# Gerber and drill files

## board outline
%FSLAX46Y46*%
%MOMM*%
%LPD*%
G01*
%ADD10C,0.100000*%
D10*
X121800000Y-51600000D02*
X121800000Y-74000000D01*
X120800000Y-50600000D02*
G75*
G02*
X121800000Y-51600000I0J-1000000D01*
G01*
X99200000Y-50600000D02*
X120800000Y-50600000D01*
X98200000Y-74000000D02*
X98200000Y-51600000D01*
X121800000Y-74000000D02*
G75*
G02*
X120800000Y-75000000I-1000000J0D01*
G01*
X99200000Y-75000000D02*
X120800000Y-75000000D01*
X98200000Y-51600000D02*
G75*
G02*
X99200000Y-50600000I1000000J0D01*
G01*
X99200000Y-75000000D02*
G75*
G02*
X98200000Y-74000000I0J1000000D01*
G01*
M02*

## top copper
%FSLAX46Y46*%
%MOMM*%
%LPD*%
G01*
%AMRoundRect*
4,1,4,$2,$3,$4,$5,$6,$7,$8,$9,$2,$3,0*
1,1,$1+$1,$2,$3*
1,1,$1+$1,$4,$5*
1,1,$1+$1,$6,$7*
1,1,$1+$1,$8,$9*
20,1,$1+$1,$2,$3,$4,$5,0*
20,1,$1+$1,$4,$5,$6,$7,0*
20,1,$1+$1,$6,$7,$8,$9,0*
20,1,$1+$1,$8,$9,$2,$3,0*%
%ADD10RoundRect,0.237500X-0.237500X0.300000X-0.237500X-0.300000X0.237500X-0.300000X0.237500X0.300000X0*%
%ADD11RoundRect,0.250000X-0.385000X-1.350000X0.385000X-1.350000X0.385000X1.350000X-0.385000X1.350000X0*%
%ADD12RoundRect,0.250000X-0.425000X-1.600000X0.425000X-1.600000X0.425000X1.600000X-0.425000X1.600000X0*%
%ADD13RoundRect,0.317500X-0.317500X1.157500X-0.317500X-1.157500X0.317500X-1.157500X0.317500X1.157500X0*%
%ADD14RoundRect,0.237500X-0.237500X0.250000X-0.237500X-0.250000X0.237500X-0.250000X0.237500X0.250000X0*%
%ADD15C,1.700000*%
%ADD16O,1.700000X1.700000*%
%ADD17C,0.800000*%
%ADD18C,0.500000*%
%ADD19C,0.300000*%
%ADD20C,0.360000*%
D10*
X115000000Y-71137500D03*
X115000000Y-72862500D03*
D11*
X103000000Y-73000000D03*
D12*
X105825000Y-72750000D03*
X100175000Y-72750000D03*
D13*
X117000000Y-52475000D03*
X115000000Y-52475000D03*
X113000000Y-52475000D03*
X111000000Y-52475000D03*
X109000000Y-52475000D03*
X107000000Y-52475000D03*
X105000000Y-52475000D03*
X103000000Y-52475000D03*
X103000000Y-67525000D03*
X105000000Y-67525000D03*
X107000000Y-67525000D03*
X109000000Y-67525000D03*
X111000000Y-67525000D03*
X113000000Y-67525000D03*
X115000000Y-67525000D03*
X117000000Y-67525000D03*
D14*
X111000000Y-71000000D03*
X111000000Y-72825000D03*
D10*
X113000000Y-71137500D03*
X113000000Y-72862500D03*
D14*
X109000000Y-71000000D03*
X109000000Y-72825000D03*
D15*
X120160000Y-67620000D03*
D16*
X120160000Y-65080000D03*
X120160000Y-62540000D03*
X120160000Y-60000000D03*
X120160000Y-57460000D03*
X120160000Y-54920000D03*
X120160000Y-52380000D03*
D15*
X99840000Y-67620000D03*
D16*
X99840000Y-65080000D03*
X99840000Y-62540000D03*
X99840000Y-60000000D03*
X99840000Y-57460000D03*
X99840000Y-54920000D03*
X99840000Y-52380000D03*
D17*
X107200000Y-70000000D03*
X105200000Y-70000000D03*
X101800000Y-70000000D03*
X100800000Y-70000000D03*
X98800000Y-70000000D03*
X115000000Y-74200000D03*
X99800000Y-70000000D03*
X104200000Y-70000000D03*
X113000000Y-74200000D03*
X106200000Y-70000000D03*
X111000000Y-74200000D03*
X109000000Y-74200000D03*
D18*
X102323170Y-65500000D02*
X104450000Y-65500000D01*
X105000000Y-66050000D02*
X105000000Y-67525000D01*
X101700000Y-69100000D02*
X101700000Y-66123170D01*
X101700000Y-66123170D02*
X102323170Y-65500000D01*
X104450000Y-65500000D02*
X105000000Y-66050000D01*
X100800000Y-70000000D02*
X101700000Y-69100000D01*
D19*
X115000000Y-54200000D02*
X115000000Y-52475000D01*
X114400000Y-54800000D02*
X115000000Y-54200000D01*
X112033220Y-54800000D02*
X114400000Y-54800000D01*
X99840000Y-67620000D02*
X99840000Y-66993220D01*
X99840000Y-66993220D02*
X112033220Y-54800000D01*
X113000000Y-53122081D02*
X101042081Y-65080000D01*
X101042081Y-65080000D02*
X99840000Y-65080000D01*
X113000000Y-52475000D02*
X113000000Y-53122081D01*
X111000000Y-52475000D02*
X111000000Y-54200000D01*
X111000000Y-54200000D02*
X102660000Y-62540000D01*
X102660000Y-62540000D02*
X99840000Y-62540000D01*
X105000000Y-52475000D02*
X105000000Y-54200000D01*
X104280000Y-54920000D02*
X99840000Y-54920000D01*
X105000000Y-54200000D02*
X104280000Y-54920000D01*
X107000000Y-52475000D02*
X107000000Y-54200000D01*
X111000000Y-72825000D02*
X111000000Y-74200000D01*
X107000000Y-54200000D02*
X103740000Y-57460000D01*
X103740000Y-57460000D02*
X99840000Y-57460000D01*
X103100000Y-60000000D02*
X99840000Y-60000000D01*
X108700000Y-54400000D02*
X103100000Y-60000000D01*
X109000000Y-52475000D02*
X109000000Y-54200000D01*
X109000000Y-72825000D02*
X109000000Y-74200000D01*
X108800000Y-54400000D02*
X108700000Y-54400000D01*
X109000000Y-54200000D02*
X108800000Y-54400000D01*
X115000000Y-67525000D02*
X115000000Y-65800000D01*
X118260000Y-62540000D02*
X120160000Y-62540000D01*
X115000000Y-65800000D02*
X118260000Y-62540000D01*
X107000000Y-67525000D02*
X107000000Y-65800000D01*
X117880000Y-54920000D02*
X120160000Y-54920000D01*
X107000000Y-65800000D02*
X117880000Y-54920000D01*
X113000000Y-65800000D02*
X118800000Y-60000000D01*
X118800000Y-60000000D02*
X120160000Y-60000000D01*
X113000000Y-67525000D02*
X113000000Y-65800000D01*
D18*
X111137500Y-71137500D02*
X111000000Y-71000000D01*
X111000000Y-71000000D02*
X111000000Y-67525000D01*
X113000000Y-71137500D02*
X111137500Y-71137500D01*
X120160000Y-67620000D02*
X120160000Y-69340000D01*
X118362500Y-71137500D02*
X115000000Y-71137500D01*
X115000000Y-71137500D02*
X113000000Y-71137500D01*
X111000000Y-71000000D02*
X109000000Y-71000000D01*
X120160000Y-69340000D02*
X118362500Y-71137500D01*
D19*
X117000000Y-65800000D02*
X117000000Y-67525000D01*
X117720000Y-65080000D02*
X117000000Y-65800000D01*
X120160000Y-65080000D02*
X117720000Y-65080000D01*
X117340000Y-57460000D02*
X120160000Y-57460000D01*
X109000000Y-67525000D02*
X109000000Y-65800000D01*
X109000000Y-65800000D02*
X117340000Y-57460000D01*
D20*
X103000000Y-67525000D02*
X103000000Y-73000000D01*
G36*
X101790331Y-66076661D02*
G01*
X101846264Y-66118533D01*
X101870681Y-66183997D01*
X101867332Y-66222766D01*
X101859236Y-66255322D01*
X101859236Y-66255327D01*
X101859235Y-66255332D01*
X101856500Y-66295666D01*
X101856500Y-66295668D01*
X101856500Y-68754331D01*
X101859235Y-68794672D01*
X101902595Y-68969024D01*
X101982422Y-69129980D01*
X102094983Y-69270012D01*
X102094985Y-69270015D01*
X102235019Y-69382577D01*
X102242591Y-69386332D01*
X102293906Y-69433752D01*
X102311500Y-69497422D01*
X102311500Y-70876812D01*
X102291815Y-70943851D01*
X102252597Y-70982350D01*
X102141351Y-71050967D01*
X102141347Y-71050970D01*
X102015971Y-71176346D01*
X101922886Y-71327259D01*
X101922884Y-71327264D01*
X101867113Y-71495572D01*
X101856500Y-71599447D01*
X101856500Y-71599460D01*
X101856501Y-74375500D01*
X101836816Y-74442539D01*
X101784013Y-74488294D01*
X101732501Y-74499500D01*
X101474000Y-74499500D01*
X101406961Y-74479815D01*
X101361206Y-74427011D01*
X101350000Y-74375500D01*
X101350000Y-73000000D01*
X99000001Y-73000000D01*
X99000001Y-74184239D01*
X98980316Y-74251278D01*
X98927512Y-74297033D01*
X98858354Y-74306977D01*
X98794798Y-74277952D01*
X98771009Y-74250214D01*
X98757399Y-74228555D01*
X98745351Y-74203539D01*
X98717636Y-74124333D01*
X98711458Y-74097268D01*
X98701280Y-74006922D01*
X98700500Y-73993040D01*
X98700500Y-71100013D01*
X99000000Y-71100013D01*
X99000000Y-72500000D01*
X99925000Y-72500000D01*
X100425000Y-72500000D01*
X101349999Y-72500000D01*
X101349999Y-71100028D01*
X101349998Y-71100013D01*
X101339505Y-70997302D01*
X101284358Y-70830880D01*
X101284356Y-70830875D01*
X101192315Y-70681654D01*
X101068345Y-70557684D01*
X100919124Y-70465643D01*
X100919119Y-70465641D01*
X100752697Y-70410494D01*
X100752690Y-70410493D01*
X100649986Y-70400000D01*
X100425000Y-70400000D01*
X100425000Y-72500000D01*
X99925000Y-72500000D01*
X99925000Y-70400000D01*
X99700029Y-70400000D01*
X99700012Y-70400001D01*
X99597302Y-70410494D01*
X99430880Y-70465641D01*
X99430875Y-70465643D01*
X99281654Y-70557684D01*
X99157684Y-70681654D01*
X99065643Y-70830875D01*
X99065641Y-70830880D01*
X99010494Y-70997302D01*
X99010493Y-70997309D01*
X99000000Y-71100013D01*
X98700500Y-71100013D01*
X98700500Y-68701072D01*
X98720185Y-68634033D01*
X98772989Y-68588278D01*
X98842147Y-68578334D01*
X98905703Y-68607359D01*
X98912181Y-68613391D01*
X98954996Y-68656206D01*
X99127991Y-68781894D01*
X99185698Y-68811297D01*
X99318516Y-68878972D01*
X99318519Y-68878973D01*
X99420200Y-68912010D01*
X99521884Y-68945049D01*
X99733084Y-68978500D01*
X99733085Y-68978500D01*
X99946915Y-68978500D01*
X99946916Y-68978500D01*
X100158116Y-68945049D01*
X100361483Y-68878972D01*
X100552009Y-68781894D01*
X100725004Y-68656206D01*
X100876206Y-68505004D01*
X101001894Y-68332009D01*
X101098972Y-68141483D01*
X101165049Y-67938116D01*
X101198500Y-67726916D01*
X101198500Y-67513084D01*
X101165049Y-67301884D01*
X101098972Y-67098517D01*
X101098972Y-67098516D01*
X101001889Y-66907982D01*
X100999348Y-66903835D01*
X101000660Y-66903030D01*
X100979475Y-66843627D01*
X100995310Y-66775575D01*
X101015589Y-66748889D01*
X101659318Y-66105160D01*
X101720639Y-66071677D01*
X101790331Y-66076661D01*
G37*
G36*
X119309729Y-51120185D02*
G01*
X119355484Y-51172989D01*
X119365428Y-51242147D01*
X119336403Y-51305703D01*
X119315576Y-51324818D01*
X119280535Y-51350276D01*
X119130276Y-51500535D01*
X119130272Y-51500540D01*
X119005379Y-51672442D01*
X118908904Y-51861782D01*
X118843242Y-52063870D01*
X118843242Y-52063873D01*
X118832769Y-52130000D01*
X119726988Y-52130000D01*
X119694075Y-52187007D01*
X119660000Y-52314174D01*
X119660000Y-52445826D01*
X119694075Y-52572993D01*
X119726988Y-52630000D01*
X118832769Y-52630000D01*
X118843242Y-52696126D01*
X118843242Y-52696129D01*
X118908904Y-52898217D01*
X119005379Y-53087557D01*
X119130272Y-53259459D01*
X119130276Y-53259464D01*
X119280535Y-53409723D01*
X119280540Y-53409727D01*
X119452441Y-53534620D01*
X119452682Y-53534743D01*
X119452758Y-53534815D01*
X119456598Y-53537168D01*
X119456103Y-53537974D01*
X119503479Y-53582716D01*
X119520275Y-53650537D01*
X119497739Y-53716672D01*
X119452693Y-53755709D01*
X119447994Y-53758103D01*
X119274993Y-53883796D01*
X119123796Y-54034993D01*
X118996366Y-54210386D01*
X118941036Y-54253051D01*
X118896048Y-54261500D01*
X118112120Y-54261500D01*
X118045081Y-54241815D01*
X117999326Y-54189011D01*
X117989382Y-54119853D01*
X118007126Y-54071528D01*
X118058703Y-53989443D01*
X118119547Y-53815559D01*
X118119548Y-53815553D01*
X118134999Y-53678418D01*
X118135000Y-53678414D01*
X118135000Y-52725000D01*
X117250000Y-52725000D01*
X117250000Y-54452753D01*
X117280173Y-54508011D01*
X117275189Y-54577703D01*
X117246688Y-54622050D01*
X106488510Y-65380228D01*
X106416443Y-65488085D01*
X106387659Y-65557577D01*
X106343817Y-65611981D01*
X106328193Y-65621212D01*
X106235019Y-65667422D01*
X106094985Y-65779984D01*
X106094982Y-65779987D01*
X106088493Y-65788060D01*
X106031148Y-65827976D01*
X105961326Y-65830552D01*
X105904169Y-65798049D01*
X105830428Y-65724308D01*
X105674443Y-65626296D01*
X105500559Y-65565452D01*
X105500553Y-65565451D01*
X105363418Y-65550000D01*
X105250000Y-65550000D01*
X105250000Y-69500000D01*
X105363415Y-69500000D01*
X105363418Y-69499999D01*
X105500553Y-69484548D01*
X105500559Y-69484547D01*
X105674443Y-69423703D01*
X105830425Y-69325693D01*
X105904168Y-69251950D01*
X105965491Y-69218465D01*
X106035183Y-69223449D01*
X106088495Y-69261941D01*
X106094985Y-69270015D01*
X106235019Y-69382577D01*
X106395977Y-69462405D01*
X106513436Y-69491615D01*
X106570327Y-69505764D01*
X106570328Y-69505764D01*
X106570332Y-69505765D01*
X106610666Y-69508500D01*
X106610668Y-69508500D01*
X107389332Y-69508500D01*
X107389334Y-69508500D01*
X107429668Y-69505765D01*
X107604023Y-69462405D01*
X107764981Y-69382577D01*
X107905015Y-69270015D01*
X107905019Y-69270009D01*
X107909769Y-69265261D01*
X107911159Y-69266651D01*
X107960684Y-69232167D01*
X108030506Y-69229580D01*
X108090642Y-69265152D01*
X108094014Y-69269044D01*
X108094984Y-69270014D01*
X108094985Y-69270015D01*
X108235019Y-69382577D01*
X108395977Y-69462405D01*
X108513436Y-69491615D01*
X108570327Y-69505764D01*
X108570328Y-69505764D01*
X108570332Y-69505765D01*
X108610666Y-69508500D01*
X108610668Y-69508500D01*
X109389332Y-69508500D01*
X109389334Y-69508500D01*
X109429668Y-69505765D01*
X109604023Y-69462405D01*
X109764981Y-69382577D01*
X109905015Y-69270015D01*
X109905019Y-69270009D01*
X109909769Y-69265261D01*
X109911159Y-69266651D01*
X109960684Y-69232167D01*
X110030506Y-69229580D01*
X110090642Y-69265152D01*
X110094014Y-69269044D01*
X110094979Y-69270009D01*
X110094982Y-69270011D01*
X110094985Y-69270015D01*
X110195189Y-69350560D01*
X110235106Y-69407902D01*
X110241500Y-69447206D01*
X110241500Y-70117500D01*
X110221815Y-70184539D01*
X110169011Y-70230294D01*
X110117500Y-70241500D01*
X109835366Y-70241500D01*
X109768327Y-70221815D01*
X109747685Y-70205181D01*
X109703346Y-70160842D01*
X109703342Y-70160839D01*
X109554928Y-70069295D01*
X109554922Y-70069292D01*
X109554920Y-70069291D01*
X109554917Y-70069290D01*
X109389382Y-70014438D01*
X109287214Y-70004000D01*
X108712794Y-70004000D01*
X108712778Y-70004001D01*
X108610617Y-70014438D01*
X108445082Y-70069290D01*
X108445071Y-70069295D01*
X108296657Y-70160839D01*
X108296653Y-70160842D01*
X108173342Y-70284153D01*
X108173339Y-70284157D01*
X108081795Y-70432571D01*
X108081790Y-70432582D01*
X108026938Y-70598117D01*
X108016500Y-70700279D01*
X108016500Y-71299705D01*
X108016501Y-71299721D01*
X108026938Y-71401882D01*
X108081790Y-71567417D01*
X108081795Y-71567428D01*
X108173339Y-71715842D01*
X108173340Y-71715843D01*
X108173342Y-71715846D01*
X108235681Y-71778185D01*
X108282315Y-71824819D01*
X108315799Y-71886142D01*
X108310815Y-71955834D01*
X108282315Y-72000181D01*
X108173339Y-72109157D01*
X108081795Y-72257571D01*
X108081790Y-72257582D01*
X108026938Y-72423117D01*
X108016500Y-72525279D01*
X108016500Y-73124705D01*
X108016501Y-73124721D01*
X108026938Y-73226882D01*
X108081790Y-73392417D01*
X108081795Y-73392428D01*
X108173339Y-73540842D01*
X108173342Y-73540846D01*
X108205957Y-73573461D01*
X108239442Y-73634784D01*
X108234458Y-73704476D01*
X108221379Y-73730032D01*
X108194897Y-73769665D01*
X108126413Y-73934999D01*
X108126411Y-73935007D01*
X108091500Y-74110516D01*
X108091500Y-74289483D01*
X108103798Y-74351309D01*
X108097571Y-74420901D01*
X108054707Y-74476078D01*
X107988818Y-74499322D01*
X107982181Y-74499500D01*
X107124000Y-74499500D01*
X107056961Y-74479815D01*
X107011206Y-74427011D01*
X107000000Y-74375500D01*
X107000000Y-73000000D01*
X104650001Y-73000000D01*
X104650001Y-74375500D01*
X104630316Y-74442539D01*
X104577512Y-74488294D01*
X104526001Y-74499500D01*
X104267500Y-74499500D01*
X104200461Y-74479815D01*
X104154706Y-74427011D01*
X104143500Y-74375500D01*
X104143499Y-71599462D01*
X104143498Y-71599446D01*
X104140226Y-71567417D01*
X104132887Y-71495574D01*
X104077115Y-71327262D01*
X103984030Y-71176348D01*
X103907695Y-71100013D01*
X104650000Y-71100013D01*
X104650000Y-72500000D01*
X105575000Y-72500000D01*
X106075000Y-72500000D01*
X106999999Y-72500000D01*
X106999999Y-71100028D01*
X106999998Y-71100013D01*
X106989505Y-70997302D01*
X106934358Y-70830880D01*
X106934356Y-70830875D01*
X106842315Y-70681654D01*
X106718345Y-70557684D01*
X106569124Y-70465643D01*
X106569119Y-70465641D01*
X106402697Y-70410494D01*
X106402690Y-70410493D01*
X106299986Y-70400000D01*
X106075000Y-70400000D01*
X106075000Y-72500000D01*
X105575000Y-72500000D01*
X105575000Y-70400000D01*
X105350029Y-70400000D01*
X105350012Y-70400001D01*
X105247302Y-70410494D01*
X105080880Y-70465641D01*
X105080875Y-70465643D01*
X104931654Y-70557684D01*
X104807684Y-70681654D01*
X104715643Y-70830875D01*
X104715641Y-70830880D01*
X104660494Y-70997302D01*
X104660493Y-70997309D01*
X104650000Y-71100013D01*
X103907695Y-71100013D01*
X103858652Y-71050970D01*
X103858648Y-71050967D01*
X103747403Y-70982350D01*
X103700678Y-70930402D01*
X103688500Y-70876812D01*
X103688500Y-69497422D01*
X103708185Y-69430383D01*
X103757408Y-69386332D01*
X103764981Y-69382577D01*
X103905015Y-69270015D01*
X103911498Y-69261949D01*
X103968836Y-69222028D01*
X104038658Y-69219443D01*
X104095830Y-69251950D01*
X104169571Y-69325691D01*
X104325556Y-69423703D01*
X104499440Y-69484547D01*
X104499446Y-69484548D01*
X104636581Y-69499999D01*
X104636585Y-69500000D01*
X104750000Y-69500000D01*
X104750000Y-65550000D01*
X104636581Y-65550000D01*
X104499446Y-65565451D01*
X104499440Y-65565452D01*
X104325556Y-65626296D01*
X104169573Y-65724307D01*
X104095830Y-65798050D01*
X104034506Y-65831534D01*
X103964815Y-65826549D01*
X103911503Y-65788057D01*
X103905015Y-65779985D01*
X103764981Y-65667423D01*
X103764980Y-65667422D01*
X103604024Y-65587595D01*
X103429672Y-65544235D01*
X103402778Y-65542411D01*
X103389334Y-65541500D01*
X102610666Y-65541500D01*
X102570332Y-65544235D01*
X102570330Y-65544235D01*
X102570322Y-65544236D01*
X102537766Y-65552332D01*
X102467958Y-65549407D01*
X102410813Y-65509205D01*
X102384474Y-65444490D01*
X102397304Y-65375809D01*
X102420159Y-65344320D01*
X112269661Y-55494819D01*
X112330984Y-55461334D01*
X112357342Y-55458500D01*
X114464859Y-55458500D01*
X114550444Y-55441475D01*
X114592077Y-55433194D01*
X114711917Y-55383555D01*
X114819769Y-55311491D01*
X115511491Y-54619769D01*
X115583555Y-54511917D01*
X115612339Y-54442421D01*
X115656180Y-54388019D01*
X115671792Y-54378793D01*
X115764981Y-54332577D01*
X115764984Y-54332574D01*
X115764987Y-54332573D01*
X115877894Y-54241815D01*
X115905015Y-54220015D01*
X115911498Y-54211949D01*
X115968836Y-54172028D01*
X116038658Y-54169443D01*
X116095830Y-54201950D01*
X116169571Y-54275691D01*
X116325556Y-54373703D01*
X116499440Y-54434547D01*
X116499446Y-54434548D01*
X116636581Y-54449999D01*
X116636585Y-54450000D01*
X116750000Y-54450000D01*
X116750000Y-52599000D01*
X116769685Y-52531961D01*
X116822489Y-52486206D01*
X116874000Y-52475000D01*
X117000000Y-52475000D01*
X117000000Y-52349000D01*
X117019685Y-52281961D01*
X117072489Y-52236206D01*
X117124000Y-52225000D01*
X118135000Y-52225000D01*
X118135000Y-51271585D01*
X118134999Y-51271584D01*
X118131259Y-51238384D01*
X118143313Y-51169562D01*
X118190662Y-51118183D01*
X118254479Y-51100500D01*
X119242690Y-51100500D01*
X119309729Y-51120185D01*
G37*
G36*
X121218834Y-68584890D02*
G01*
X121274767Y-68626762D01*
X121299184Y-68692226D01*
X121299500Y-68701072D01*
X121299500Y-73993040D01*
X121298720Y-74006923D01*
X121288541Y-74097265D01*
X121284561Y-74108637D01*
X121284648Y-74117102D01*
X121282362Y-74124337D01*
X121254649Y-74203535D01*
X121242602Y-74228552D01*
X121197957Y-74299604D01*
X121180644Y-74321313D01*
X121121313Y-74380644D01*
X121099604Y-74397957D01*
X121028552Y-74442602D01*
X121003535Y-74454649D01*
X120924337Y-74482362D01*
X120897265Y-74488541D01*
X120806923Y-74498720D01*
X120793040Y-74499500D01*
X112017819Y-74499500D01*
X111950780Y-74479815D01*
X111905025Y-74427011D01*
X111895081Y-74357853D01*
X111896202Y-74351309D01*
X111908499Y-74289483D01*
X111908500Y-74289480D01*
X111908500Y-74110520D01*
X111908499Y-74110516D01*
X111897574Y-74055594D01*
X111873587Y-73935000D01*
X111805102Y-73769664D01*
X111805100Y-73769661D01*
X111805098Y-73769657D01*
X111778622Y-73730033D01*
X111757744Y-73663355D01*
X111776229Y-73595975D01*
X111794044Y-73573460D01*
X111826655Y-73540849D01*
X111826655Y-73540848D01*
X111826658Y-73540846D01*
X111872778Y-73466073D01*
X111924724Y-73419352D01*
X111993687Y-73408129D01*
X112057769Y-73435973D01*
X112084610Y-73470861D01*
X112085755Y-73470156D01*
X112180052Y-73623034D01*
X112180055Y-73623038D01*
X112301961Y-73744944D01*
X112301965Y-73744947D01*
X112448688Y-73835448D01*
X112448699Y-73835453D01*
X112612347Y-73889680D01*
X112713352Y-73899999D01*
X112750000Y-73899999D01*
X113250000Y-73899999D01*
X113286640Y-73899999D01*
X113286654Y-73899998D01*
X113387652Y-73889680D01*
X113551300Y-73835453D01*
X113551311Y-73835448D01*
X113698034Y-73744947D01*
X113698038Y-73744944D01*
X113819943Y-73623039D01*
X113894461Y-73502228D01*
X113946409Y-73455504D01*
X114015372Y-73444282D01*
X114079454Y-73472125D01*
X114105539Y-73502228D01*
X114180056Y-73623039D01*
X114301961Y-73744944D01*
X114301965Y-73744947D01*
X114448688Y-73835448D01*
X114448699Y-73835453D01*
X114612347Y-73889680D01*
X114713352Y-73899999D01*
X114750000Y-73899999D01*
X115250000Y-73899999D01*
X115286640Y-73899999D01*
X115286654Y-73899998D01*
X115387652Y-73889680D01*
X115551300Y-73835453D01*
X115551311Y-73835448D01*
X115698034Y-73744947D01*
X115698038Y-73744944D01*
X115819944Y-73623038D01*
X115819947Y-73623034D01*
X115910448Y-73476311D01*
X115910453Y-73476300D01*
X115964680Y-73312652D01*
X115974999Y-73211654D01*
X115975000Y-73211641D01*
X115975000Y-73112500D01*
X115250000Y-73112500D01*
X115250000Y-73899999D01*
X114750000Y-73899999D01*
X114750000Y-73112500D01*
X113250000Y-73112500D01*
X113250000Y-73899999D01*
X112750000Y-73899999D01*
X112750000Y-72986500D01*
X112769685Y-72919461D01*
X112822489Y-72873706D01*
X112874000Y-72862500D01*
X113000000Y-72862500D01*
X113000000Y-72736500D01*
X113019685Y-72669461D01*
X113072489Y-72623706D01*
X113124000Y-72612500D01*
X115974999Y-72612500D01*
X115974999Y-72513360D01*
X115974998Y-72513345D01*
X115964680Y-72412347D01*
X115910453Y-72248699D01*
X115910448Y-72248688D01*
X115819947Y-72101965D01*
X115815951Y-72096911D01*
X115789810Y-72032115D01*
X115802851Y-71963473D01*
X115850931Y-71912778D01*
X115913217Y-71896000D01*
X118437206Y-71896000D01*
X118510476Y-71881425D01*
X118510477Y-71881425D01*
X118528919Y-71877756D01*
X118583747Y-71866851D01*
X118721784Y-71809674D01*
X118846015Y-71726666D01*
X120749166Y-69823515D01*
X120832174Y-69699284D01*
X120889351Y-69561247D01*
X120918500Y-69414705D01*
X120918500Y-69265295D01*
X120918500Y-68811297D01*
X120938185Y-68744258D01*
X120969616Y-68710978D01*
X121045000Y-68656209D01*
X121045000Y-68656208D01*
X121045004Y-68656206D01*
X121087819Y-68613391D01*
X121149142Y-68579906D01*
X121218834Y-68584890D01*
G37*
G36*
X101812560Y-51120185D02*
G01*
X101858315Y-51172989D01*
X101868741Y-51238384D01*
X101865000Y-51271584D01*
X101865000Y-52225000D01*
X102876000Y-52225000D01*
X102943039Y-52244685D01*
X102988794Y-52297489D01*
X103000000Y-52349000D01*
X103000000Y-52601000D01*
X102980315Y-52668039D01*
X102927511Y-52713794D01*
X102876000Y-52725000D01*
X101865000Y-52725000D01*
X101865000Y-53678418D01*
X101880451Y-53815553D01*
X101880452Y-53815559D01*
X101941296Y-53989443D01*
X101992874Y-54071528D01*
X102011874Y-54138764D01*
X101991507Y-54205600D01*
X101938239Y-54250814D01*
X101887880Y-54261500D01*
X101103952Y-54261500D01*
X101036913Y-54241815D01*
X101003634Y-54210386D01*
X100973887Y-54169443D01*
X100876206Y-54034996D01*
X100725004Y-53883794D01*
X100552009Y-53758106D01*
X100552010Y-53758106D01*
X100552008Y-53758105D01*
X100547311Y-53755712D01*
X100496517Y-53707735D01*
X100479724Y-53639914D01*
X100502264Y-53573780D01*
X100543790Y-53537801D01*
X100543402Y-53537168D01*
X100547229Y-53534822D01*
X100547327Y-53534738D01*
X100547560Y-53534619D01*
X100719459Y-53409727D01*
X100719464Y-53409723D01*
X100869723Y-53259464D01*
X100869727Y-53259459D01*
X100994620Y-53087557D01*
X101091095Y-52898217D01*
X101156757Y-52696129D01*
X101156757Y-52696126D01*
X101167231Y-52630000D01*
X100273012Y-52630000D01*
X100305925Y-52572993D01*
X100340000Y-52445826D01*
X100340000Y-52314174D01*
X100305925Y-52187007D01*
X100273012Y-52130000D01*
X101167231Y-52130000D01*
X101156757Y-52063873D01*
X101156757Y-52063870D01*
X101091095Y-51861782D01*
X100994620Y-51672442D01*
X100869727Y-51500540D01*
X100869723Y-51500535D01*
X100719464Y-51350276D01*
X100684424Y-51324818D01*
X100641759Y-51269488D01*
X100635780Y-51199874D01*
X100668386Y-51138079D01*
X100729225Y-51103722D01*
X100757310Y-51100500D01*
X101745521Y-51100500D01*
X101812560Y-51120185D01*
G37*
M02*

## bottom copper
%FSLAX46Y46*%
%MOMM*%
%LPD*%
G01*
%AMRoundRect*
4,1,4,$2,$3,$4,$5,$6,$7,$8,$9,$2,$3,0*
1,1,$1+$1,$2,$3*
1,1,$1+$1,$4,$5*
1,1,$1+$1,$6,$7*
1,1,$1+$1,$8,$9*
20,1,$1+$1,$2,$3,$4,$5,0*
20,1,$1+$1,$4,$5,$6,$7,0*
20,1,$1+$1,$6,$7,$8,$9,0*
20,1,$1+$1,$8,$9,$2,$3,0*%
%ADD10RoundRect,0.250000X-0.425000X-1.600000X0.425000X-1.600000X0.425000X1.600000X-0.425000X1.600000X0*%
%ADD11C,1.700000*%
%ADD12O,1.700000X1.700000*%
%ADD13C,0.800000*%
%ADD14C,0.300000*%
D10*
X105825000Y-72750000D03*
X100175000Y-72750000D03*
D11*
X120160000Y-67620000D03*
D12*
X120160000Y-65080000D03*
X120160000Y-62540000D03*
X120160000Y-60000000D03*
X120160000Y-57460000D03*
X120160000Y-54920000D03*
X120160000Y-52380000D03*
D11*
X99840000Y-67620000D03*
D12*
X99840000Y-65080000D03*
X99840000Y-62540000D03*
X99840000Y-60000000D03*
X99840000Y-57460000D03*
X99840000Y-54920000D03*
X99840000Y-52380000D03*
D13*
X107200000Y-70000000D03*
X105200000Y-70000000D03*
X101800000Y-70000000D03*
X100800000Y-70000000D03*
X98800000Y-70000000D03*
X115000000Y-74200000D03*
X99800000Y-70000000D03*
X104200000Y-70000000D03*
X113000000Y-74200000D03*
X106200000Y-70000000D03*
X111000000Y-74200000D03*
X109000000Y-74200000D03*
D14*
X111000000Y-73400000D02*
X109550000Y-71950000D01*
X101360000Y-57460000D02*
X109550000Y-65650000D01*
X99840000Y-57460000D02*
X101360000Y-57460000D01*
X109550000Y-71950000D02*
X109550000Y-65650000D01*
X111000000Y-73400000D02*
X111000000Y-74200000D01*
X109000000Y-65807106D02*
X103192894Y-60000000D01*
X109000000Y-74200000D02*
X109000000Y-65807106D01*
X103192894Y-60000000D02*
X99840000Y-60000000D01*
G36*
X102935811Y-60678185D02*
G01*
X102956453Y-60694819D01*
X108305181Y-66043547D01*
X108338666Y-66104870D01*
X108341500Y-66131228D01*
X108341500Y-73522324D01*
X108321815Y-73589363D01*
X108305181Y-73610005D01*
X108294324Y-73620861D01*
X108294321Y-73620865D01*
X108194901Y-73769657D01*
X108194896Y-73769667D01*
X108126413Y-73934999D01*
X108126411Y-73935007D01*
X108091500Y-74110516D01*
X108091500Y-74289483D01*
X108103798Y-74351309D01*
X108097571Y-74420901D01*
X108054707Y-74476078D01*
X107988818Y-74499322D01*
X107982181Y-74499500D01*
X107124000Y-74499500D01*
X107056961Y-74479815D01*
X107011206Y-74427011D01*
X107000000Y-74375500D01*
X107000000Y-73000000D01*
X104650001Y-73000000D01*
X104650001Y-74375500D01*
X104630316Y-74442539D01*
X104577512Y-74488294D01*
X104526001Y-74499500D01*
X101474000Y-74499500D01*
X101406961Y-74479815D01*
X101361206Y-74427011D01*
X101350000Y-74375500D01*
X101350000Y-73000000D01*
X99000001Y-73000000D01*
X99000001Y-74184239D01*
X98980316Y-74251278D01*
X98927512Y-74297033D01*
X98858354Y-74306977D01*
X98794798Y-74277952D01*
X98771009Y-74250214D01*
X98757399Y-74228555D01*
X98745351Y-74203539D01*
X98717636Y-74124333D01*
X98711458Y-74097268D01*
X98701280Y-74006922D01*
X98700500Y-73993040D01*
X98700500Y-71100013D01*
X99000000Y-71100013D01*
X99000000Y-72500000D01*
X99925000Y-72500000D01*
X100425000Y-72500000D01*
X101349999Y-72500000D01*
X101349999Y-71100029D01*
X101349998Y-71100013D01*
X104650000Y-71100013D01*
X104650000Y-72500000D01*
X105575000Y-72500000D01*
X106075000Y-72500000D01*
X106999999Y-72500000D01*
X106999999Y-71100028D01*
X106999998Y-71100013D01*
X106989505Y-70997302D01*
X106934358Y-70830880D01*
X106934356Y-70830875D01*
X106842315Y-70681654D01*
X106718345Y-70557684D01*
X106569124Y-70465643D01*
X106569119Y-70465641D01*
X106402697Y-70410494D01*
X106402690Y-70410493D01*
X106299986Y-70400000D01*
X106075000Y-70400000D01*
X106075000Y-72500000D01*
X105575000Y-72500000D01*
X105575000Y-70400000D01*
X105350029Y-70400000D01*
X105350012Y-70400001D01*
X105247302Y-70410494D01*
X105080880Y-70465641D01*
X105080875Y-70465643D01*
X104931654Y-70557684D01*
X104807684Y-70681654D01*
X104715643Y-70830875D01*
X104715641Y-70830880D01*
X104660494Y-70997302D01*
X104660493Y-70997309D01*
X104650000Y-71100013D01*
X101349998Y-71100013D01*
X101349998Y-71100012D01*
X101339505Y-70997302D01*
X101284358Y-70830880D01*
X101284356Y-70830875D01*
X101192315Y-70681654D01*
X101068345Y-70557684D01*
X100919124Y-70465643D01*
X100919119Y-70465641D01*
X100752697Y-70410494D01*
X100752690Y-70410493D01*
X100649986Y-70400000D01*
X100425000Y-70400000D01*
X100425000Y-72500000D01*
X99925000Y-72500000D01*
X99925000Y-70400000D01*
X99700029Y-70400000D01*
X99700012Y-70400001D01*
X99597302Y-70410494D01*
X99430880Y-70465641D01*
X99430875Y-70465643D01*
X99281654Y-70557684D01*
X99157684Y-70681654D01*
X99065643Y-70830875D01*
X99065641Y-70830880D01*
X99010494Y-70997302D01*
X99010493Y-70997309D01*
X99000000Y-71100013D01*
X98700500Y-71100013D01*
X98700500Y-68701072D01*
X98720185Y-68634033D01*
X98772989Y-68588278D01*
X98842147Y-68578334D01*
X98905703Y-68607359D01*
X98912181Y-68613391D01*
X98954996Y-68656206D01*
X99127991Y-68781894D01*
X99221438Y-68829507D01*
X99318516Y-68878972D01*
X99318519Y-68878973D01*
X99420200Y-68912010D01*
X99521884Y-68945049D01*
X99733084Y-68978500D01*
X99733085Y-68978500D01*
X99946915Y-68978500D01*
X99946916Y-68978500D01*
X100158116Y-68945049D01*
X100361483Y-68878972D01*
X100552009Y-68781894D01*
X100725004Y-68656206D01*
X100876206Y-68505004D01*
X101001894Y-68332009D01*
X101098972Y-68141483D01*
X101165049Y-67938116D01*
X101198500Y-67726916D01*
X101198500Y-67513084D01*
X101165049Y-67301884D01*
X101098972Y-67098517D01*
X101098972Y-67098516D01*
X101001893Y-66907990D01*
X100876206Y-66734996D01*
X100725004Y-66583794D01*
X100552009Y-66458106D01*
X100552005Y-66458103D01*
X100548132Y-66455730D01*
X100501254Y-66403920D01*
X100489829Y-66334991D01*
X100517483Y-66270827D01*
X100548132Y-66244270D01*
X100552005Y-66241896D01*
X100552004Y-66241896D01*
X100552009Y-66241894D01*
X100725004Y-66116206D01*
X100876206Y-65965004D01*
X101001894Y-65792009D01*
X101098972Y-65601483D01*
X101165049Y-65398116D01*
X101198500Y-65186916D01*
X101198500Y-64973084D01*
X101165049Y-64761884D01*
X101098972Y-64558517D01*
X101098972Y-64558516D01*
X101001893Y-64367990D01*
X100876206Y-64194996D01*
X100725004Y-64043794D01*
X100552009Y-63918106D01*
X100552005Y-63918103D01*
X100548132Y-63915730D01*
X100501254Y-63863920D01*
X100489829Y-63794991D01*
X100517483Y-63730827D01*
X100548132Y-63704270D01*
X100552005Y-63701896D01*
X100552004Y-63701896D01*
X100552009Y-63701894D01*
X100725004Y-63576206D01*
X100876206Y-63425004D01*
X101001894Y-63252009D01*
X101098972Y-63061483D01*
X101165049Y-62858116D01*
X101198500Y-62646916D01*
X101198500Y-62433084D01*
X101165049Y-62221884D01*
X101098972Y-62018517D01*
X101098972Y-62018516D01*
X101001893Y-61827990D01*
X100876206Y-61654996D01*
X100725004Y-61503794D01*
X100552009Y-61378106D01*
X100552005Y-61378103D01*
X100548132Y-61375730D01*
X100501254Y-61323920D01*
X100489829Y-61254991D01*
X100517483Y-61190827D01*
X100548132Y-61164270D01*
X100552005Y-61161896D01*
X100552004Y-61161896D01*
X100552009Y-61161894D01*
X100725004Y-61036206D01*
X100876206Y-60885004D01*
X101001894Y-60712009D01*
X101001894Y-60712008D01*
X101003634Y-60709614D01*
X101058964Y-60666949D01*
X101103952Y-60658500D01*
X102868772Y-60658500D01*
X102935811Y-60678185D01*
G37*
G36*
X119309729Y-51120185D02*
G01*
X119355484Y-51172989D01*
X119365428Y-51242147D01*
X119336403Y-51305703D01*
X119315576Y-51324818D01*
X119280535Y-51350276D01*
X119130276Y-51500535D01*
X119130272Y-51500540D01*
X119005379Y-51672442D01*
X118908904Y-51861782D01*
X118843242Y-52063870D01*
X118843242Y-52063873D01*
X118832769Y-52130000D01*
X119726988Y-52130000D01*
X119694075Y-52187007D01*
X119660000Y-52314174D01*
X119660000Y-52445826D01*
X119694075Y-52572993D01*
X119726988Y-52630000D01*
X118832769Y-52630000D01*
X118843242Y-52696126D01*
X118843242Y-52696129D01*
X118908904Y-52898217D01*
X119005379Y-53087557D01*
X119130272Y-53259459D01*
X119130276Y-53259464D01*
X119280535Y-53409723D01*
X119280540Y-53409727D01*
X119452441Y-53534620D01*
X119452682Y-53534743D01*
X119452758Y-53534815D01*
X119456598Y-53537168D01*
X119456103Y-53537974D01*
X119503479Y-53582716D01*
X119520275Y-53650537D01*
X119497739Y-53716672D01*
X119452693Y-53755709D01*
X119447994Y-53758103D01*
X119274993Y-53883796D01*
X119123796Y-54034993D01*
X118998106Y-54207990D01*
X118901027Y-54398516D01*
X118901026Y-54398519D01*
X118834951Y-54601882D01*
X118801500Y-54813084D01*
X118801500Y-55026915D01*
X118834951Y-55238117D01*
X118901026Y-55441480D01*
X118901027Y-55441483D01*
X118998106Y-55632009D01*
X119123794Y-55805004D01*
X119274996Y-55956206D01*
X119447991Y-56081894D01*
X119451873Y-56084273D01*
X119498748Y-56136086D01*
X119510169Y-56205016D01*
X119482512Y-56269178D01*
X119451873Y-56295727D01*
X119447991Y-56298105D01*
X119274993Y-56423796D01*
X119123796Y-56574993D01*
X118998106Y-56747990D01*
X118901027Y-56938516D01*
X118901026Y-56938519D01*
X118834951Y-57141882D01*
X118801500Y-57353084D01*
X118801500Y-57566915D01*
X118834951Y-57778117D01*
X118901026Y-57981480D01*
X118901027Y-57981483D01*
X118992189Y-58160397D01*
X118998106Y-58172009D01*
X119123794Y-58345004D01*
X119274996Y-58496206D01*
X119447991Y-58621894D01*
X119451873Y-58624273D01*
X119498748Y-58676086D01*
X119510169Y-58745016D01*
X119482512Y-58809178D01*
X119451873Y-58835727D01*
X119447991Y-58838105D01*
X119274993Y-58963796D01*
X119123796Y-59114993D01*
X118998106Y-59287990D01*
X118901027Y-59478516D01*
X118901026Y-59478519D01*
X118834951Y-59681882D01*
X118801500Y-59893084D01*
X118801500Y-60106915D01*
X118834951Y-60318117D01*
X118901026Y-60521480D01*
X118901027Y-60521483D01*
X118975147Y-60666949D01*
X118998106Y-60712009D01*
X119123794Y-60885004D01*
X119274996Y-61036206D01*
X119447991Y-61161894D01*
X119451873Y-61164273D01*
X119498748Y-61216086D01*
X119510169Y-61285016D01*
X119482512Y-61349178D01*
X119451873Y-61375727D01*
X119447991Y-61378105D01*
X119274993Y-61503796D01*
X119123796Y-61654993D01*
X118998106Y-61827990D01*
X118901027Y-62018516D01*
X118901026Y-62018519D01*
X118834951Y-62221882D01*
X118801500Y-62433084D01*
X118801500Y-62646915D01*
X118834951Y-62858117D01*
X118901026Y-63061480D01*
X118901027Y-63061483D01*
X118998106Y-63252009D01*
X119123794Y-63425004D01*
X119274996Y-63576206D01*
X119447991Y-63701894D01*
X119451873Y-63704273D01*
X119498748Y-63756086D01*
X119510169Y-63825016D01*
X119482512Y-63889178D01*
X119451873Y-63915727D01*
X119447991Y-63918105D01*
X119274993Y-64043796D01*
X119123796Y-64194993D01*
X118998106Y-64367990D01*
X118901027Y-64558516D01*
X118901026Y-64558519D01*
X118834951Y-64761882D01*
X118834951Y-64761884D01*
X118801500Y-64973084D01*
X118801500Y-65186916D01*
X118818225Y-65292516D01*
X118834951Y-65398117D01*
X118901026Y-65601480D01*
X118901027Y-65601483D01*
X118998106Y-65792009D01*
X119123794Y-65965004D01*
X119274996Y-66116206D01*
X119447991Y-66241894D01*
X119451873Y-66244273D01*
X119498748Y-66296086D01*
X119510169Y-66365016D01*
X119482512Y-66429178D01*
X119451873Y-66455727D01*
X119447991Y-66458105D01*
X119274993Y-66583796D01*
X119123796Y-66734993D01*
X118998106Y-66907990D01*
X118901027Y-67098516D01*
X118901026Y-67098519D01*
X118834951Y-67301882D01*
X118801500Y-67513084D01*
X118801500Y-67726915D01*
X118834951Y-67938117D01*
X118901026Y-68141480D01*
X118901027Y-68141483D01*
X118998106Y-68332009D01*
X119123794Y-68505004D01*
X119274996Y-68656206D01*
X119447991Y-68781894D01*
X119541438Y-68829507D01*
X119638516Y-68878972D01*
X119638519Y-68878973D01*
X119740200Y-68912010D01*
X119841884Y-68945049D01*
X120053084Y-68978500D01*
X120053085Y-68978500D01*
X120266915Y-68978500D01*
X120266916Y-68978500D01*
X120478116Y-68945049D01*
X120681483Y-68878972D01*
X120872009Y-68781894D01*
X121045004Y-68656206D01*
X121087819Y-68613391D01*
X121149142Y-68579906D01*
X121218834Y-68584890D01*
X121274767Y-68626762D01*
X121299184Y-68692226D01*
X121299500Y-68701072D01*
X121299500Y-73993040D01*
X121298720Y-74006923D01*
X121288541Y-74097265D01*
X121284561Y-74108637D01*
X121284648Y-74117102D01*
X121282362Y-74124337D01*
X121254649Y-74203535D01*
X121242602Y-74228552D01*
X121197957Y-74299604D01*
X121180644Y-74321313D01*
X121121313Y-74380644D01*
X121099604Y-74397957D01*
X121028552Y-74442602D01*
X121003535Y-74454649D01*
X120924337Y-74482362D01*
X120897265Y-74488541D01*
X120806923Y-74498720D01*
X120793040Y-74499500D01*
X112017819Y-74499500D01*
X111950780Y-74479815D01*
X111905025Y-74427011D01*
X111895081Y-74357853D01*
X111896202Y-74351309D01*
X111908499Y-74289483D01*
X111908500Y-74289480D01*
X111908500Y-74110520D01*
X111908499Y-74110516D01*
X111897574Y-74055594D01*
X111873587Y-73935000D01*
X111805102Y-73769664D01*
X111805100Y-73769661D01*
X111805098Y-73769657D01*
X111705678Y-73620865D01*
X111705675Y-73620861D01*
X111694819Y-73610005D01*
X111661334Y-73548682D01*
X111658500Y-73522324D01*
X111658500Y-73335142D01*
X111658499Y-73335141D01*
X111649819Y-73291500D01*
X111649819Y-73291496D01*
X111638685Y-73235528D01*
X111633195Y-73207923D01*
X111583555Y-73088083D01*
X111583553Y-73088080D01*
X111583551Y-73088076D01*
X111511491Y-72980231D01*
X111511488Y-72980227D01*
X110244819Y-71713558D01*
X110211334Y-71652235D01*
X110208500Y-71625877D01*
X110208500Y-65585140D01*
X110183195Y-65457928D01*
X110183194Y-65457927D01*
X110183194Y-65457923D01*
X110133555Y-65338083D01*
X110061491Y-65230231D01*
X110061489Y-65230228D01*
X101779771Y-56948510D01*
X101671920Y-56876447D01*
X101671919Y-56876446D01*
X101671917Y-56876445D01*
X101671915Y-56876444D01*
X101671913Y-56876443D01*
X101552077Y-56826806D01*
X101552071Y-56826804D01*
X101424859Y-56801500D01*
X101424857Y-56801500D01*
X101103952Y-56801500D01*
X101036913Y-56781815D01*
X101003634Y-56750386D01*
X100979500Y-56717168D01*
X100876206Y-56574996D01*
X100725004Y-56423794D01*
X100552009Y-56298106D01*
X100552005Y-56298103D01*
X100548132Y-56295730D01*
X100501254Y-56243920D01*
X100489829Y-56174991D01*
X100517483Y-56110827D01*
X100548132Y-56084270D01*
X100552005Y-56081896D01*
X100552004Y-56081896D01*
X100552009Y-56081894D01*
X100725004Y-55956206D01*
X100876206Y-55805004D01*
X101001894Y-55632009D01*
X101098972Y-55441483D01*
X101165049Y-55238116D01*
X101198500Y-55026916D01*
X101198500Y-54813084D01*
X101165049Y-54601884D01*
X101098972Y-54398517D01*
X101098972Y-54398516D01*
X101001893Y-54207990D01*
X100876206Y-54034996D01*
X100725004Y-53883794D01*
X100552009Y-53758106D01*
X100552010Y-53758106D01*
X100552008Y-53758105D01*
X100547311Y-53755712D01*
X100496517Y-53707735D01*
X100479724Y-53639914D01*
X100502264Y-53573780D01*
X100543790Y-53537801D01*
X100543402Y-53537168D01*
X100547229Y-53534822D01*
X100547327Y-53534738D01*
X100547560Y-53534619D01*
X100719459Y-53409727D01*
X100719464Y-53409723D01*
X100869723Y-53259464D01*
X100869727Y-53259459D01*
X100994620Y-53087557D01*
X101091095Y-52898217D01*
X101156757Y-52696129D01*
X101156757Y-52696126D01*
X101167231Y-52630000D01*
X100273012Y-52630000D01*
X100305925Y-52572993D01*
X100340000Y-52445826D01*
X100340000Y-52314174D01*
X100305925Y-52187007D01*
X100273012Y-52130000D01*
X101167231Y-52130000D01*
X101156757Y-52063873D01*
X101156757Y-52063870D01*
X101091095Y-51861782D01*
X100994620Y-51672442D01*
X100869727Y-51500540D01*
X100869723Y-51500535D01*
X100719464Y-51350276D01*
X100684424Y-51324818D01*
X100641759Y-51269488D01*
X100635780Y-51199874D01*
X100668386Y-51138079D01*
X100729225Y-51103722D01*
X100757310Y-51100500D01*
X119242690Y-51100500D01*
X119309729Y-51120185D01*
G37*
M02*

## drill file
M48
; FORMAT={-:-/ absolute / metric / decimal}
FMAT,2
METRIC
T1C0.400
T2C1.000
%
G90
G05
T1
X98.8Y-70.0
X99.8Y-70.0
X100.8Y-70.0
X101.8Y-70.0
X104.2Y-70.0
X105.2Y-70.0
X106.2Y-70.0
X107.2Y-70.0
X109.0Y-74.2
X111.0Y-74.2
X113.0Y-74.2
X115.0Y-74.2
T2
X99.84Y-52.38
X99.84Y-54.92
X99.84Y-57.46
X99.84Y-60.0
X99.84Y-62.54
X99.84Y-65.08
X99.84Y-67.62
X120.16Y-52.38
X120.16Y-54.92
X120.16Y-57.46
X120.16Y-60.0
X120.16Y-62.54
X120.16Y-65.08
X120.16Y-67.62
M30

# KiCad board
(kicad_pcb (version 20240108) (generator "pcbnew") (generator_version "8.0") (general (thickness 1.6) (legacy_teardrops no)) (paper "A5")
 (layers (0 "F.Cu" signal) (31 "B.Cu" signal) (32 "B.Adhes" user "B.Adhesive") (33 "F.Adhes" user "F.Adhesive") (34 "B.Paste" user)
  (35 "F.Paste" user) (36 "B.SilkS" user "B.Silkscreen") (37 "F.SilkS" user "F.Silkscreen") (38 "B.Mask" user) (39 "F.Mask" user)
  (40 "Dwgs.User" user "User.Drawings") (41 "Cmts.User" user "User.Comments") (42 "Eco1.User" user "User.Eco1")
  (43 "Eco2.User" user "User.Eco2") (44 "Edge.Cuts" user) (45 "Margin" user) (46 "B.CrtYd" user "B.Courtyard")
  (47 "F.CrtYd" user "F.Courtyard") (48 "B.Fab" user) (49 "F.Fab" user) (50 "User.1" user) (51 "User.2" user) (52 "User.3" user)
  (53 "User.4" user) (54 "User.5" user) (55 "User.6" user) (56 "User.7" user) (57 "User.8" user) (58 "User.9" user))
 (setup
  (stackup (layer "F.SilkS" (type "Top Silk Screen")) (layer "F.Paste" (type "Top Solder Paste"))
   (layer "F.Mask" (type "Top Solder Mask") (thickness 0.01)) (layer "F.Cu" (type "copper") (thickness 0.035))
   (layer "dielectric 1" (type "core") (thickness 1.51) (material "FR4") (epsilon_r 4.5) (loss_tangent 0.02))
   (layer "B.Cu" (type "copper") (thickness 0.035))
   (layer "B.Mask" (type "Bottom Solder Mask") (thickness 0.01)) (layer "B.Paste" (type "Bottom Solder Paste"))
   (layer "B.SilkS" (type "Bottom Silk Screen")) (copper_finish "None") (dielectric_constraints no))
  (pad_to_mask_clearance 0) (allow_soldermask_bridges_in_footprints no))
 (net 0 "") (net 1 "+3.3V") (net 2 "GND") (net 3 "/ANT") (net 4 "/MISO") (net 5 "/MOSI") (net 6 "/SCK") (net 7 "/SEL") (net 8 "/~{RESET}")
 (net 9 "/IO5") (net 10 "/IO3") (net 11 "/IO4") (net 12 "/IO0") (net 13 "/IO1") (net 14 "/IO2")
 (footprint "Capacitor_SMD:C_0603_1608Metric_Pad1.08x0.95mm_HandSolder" (layer "F.Cu") (at 115 72 -90)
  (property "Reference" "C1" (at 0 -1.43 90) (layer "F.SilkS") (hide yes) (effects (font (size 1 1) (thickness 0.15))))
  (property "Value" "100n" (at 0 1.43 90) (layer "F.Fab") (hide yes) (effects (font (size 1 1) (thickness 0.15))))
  (pad "1" smd roundrect (at -0.8625 0 270) (size 1.075 0.95) (layers "F.Cu" "F.Paste" "F.Mask") (roundrect_rratio 0.25) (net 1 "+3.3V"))
  (pad "2" smd roundrect (at 0.8625 0 270) (size 1.075 0.95) (layers "F.Cu" "F.Paste" "F.Mask") (roundrect_rratio 0.25) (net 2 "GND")))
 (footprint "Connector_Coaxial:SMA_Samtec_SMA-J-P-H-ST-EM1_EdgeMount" (layer "F.Cu") (at 103 73 -90)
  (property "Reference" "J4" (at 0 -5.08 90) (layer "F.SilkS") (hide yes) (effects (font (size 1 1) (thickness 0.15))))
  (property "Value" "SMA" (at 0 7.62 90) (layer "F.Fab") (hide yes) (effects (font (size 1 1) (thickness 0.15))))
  (pad "1" smd roundrect (at 0 0) (size 1.27 3.2) (layers "F.Cu" "F.Mask") (roundrect_rratio 0.1968503937) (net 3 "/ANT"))
  (pad "2" smd roundrect (at -0.25 -2.825) (size 1.35 3.7) (layers "F.Cu" "F.Mask") (roundrect_rratio 0.1851851852) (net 2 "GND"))
  (pad "2" smd roundrect (at -0.25 -2.825) (size 1.35 3.7) (layers "B.Cu" "B.Mask") (roundrect_rratio 0.1851851852) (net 2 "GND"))
  (pad "2" smd roundrect (at -0.25 2.825) (size 1.35 3.7) (layers "F.Cu" "F.Mask") (roundrect_rratio 0.1851851852) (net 2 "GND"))
  (pad "2" smd roundrect (at -0.25 2.825) (size 1.35 3.7) (layers "B.Cu" "B.Mask") (roundrect_rratio 0.1851851852) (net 2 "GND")))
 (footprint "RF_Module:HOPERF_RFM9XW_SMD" (layer "F.Cu") (at 110 60 -90)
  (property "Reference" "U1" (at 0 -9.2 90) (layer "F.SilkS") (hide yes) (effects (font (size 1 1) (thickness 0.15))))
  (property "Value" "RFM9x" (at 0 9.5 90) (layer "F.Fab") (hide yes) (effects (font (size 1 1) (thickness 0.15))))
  (pad "1" smd roundrect (at -7.525 -7 270) (size 2.95 1.27) (layers "F.Cu" "F.Paste" "F.Mask") (roundrect_rratio 0.25) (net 2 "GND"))
  (pad "2" smd roundrect (at -7.525 -5 270) (size 2.95 1.27) (layers "F.Cu" "F.Paste" "F.Mask") (roundrect_rratio 0.25) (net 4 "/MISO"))
  (pad "3" smd roundrect (at -7.525 -3 270) (size 2.95 1.27) (layers "F.Cu" "F.Paste" "F.Mask") (roundrect_rratio 0.25) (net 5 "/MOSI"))
  (pad "4" smd roundrect (at -7.525 -1 270) (size 2.95 1.27) (layers "F.Cu" "F.Paste" "F.Mask") (roundrect_rratio 0.25) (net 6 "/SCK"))
  (pad "5" smd roundrect (at -7.525 1 270) (size 2.95 1.27) (layers "F.Cu" "F.Paste" "F.Mask") (roundrect_rratio 0.25) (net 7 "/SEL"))
  (pad "6" smd roundrect (at -7.525 3 270) (size 2.95 1.27) (layers "F.Cu" "F.Paste" "F.Mask") (roundrect_rratio 0.25) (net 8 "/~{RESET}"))
  (pad "7" smd roundrect (at -7.525 5 270) (size 2.95 1.27) (layers "F.Cu" "F.Paste" "F.Mask") (roundrect_rratio 0.25) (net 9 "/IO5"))
  (pad "8" smd roundrect (at -7.525 7 270) (size 2.95 1.27) (layers "F.Cu" "F.Paste" "F.Mask") (roundrect_rratio 0.25) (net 2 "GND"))
  (pad "9" smd roundrect (at 7.525 7 270) (size 2.95 1.27) (layers "F.Cu" "F.Paste" "F.Mask") (roundrect_rratio 0.25) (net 3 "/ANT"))
  (pad "10" smd roundrect (at 7.525 5 270) (size 2.95 1.27) (layers "F.Cu" "F.Paste" "F.Mask") (roundrect_rratio 0.25) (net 2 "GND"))
  (pad "11" smd roundrect (at 7.525 3 270) (size 2.95 1.27) (layers "F.Cu" "F.Paste" "F.Mask") (roundrect_rratio 0.25) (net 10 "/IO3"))
  (pad "12" smd roundrect (at 7.525 1 270) (size 2.95 1.27) (layers "F.Cu" "F.Paste" "F.Mask") (roundrect_rratio 0.25) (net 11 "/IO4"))
  (pad "13" smd roundrect (at 7.525 -1 270) (size 2.95 1.27) (layers "F.Cu" "F.Paste" "F.Mask") (roundrect_rratio 0.25) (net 1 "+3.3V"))
  (pad "14" smd roundrect (at 7.525 -3 270) (size 2.95 1.27) (layers "F.Cu" "F.Paste" "F.Mask") (roundrect_rratio 0.25) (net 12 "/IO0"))
  (pad "15" smd roundrect (at 7.525 -5 270) (size 2.95 1.27) (layers "F.Cu" "F.Paste" "F.Mask") (roundrect_rratio 0.25) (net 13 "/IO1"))
  (pad "16" smd roundrect (at 7.525 -7 270) (size 2.95 1.27) (layers "F.Cu" "F.Paste" "F.Mask") (roundrect_rratio 0.25) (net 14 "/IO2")))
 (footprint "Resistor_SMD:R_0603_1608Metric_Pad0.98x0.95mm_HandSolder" (layer "F.Cu") (at 111 71.9125 -90)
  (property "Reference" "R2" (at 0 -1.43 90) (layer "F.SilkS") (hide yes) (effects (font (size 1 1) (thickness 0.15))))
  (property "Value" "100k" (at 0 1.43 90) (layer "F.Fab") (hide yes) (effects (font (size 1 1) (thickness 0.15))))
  (pad "1" smd roundrect (at -0.9125 0 270) (size 0.975 0.95) (layers "F.Cu" "F.Paste" "F.Mask") (roundrect_rratio 0.25) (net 1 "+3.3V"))
  (pad "2" smd roundrect (at 0.9125 0 270) (size 0.975 0.95) (layers "F.Cu" "F.Paste" "F.Mask") (roundrect_rratio 0.25) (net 8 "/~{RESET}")))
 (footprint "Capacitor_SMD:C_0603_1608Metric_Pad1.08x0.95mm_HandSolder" (layer "F.Cu") (at 113 72 -90)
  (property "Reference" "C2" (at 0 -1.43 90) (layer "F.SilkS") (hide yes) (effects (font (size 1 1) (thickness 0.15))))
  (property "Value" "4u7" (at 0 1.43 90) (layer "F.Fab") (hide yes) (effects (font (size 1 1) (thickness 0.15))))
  (pad "1" smd roundrect (at -0.8625 0 270) (size 1.075 0.95) (layers "F.Cu" "F.Paste" "F.Mask") (roundrect_rratio 0.25) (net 1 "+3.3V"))
  (pad "2" smd roundrect (at 0.8625 0 270) (size 1.075 0.95) (layers "F.Cu" "F.Paste" "F.Mask") (roundrect_rratio 0.25) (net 2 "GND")))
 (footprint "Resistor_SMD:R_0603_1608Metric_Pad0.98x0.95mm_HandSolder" (layer "F.Cu") (at 109 71.9125 -90)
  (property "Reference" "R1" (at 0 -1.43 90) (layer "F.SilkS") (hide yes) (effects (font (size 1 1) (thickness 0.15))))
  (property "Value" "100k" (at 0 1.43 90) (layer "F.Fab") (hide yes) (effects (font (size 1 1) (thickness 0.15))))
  (pad "1" smd roundrect (at -0.9125 0 270) (size 0.975 0.95) (layers "F.Cu" "F.Paste" "F.Mask") (roundrect_rratio 0.25) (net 1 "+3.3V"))
  (pad "2" smd roundrect (at 0.9125 0 270) (size 0.975 0.95) (layers "F.Cu" "F.Paste" "F.Mask") (roundrect_rratio 0.25) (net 7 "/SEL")))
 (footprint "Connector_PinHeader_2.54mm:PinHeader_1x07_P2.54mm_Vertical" (layer "B.Cu") (at 120.16 67.62)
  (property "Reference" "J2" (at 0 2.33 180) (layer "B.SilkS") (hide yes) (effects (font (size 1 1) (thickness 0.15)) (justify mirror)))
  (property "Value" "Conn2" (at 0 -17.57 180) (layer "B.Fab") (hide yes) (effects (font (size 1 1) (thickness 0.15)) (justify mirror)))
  (pad "1" thru_hole circle (at 0 0) (size 1.7 1.7) (drill 1) (layers "*.Cu" "*.Mask") (remove_unused_layers no) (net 1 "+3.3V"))
  (pad "2" thru_hole oval (at 0 -2.54) (size 1.7 1.7) (drill 1) (layers "*.Cu" "*.Mask") (remove_unused_layers no) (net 14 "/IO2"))
  (pad "3" thru_hole oval (at 0 -5.08) (size 1.7 1.7) (drill 1) (layers "*.Cu" "*.Mask") (remove_unused_layers no) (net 13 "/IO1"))
  (pad "4" thru_hole oval (at 0 -7.62) (size 1.7 1.7) (drill 1) (layers "*.Cu" "*.Mask") (remove_unused_layers no) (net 12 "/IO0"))
  (pad "5" thru_hole oval (at 0 -10.16) (size 1.7 1.7) (drill 1) (layers "*.Cu" "*.Mask") (remove_unused_layers no) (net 11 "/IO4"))
  (pad "6" thru_hole oval (at 0 -12.7) (size 1.7 1.7) (drill 1) (layers "*.Cu" "*.Mask") (remove_unused_layers no) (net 10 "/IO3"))
  (pad "7" thru_hole oval (at 0 -15.24) (size 1.7 1.7) (drill 1) (layers "*.Cu" "*.Mask") (remove_unused_layers no) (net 2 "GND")))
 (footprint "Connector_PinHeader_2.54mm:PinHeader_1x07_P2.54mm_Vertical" (layer "B.Cu") (at 99.84 67.62)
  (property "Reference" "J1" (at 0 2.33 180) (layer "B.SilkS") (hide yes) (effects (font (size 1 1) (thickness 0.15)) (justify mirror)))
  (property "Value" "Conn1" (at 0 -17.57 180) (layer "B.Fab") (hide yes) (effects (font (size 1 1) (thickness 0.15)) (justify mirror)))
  (pad "1" thru_hole circle (at 0 0) (size 1.7 1.7) (drill 1) (layers "*.Cu" "*.Mask") (remove_unused_layers no) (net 4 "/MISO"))
  (pad "2" thru_hole oval (at 0 -2.54) (size 1.7 1.7) (drill 1) (layers "*.Cu" "*.Mask") (remove_unused_layers no) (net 5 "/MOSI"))
  (pad "3" thru_hole oval (at 0 -5.08) (size 1.7 1.7) (drill 1) (layers "*.Cu" "*.Mask") (remove_unused_layers no) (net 6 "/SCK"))
  (pad "4" thru_hole oval (at 0 -7.62) (size 1.7 1.7) (drill 1) (layers "*.Cu" "*.Mask") (remove_unused_layers no) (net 7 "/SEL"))
  (pad "5" thru_hole oval (at 0 -10.16) (size 1.7 1.7) (drill 1) (layers "*.Cu" "*.Mask") (remove_unused_layers no) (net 8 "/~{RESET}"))
  (pad "6" thru_hole oval (at 0 -12.7) (size 1.7 1.7) (drill 1) (layers "*.Cu" "*.Mask") (remove_unused_layers no) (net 9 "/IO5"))
  (pad "7" thru_hole oval (at 0 -15.24) (size 1.7 1.7) (drill 1) (layers "*.Cu" "*.Mask") (remove_unused_layers no) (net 2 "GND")))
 (gr_line (start 121.8 51.6) (end 121.8 74) (stroke (width 0.1) (type default)) (layer "Edge.Cuts"))
 (gr_arc (start 120.8 50.6) (mid 121.507107 50.892893) (end 121.8 51.6) (stroke (width 0.1) (type default)) (layer "Edge.Cuts"))
 (gr_line (start 99.2 50.6) (end 120.8 50.6) (stroke (width 0.1) (type default)) (layer "Edge.Cuts"))
 (gr_line (start 98.2 74) (end 98.2 51.6) (stroke (width 0.1) (type default)) (layer "Edge.Cuts"))
 (gr_arc (start 121.8 74) (mid 121.507107 74.707107) (end 120.8 75) (stroke (width 0.1) (type default)) (layer "Edge.Cuts"))
 (gr_line (start 99.2 75) (end 120.8 75) (stroke (width 0.1) (type default)) (layer "Edge.Cuts"))
 (gr_arc (start 98.2 51.6) (mid 98.492893 50.892893) (end 99.2 50.6) (stroke (width 0.1) (type default)) (layer "Edge.Cuts"))
 (gr_arc (start 99.2 75) (mid 98.492893 74.707107) (end 98.2 74) (stroke (width 0.1) (type default)) (layer "Edge.Cuts"))
 (segment (start 102.32317 65.5) (end 104.45 65.5) (width 0.5) (layer "F.Cu") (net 2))
 (segment (start 105 66.05) (end 105 67.525) (width 0.5) (layer "F.Cu") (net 2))
 (segment (start 101.7 69.1) (end 101.7 66.12317) (width 0.5) (layer "F.Cu") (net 2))
 (segment (start 101.7 66.12317) (end 102.32317 65.5) (width 0.5) (layer "F.Cu") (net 2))
 (segment (start 104.45 65.5) (end 105 66.05) (width 0.5) (layer "F.Cu") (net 2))
 (segment (start 100.8 70) (end 101.7 69.1) (width 0.5) (layer "F.Cu") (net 2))
 (via (at 107.2 70) (size 0.8) (drill 0.4) (layers "F.Cu" "B.Cu") (free yes) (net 2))
 (via (at 105.2 70) (size 0.8) (drill 0.4) (layers "F.Cu" "B.Cu") (free yes) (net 2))
 (via (at 101.8 70) (size 0.8) (drill 0.4) (layers "F.Cu" "B.Cu") (free yes) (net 2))
 (via (at 100.8 70) (size 0.8) (drill 0.4) (layers "F.Cu" "B.Cu") (free yes) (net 2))
 (via (at 98.8 70) (size 0.8) (drill 0.4) (layers "F.Cu" "B.Cu") (free yes) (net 2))
 (via (at 115 74.2) (size 0.8) (drill 0.4) (layers "F.Cu" "B.Cu") (free yes) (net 2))
 (via (at 99.8 70) (size 0.8) (drill 0.4) (layers "F.Cu" "B.Cu") (free yes) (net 2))
 (via (at 104.2 70) (size 0.8) (drill 0.4) (layers "F.Cu" "B.Cu") (free yes) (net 2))
 (via (at 113 74.2) (size 0.8) (drill 0.4) (layers "F.Cu" "B.Cu") (free yes) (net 2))
 (via (at 106.2 70) (size 0.8) (drill 0.4) (layers "F.Cu" "B.Cu") (free yes) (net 2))
 (segment (start 115 54.2) (end 115 52.475) (width 0.3) (layer "F.Cu") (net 4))
 (segment (start 114.4 54.8) (end 115 54.2) (width 0.3) (layer "F.Cu") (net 4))
 (segment (start 112.03322 54.8) (end 114.4 54.8) (width 0.3) (layer "F.Cu") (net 4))
 (segment (start 99.84 67.62) (end 99.84 66.99322) (width 0.3) (layer "F.Cu") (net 4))
 (segment (start 99.84 66.99322) (end 112.03322 54.8) (width 0.3) (layer "F.Cu") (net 4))
 (segment (start 113 53.122081) (end 101.042081 65.08) (width 0.3) (layer "F.Cu") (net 5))
 (segment (start 101.042081 65.08) (end 99.84 65.08) (width 0.3) (layer "F.Cu") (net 5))
 (segment (start 113 52.475) (end 113 53.122081) (width 0.3) (layer "F.Cu") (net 5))
 (segment (start 111 52.475) (end 111 54.2) (width 0.3) (layer "F.Cu") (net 6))
 (segment (start 111 54.2) (end 102.66 62.54) (width 0.3) (layer "F.Cu") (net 6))
 (segment (start 102.66 62.54) (end 99.84 62.54) (width 0.3) (layer "F.Cu") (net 6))
 (segment (start 105 52.475) (end 105 54.2) (width 0.3) (layer "F.Cu") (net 9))
 (segment (start 104.28 54.92) (end 99.84 54.92) (width 0.3) (layer "F.Cu") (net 9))
 (segment (start 105 54.2) (end 104.28 54.92) (width 0.3) (layer "F.Cu") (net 9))
 (segment (start 107 52.475) (end 107 54.2) (width 0.3) (layer "F.Cu") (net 8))
 (segment (start 111 72.825) (end 111 74.2) (width 0.3) (layer "F.Cu") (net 8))
 (segment (start 107 54.2) (end 103.74 57.46) (width 0.3) (layer "F.Cu") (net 8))
 (segment (start 103.74 57.46) (end 99.84 57.46) (width 0.3) (layer "F.Cu") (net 8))
 (via (at 111 74.2) (size 0.8) (drill 0.4) (layers "F.Cu" "B.Cu") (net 8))
 (segment (start 111 73.4) (end 109.55 71.95) (width 0.3) (layer "B.Cu") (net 8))
 (segment (start 101.36 57.46) (end 109.55 65.65) (width 0.3) (layer "B.Cu") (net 8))
 (segment (start 99.84 57.46) (end 101.36 57.46) (width 0.3) (layer "B.Cu") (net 8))
 (segment (start 109.55 71.95) (end 109.55 65.65) (width 0.3) (layer "B.Cu") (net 8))
 (segment (start 111 73.4) (end 111 74.2) (width 0.3) (layer "B.Cu") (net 8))
 (segment (start 103.1 60) (end 99.84 60) (width 0.3) (layer "F.Cu") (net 7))
 (segment (start 108.7 54.4) (end 103.1 60) (width 0.3) (layer "F.Cu") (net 7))
 (segment (start 109 52.475) (end 109 54.2) (width 0.3) (layer "F.Cu") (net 7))
 (segment (start 109 72.825) (end 109 74.2) (width 0.3) (layer "F.Cu") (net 7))
 (segment (start 108.8 54.4) (end 108.7 54.4) (width 0.3) (layer "F.Cu") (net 7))
 (segment (start 109 54.2) (end 108.8 54.4) (width 0.3) (layer "F.Cu") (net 7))
 (via (at 109 74.2) (size 0.8) (drill 0.4) (layers "F.Cu" "B.Cu") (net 7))
 (segment (start 109 65.807106) (end 103.192894 60) (width 0.3) (layer "B.Cu") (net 7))
 (segment (start 109 74.2) (end 109 65.807106) (width 0.3) (layer "B.Cu") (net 7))
 (segment (start 103.192894 60) (end 99.84 60) (width 0.3) (layer "B.Cu") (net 7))
 (segment (start 115 67.525) (end 115 65.8) (width 0.3) (layer "F.Cu") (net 13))
 (segment (start 118.26 62.54) (end 120.16 62.54) (width 0.3) (layer "F.Cu") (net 13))
 (segment (start 115 65.8) (end 118.26 62.54) (width 0.3) (layer "F.Cu") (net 13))
 (segment (start 107 67.525) (end 107 65.8) (width 0.3) (layer "F.Cu") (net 10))
 (segment (start 117.88 54.92) (end 120.16 54.92) (width 0.3) (layer "F.Cu") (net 10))
 (segment (start 107 65.8) (end 117.88 54.92) (width 0.3) (layer "F.Cu") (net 10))
 (segment (start 113 65.8) (end 118.8 60) (width 0.3) (layer "F.Cu") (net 12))
 (segment (start 118.8 60) (end 120.16 60) (width 0.3) (layer "F.Cu") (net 12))
 (segment (start 113 67.525) (end 113 65.8) (width 0.3) (layer "F.Cu") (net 12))
 (segment (start 111.1375 71.1375) (end 111 71) (width 0.5) (layer "F.Cu") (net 1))
 (segment (start 111 71) (end 111 67.525) (width 0.5) (layer "F.Cu") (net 1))
 (segment (start 113 71.1375) (end 111.1375 71.1375) (width 0.5) (layer "F.Cu") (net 1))
 (segment (start 120.16 67.62) (end 120.16 69.34) (width 0.5) (layer "F.Cu") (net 1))
 (segment (start 118.3625 71.1375) (end 115 71.1375) (width 0.5) (layer "F.Cu") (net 1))
 (segment (start 115 71.1375) (end 113 71.1375) (width 0.5) (layer "F.Cu") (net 1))
 (segment (start 111 71) (end 109 71) (width 0.5) (layer "F.Cu") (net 1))
 (segment (start 120.16 69.34) (end 118.3625 71.1375) (width 0.5) (layer "F.Cu") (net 1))
 (segment (start 117 65.8) (end 117 67.525) (width 0.3) (layer "F.Cu") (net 14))
 (segment (start 117.72 65.08) (end 117 65.8) (width 0.3) (layer "F.Cu") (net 14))
 (segment (start 120.16 65.08) (end 117.72 65.08) (width 0.3) (layer "F.Cu") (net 14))
 (segment (start 117.34 57.46) (end 120.16 57.46) (width 0.3) (layer "F.Cu") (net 11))
 (segment (start 109 67.525) (end 109 65.8) (width 0.3) (layer "F.Cu") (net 11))
 (segment (start 109 65.8) (end 117.34 57.46) (width 0.3) (layer "F.Cu") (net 11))
 (segment (start 103 67.525) (end 103 73) (width 0.36) (layer "F.Cu") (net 3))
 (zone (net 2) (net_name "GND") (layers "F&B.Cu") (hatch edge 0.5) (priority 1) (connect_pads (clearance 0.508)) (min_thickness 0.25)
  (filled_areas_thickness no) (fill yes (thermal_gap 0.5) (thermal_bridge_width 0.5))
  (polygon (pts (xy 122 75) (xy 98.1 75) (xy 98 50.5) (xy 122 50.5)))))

